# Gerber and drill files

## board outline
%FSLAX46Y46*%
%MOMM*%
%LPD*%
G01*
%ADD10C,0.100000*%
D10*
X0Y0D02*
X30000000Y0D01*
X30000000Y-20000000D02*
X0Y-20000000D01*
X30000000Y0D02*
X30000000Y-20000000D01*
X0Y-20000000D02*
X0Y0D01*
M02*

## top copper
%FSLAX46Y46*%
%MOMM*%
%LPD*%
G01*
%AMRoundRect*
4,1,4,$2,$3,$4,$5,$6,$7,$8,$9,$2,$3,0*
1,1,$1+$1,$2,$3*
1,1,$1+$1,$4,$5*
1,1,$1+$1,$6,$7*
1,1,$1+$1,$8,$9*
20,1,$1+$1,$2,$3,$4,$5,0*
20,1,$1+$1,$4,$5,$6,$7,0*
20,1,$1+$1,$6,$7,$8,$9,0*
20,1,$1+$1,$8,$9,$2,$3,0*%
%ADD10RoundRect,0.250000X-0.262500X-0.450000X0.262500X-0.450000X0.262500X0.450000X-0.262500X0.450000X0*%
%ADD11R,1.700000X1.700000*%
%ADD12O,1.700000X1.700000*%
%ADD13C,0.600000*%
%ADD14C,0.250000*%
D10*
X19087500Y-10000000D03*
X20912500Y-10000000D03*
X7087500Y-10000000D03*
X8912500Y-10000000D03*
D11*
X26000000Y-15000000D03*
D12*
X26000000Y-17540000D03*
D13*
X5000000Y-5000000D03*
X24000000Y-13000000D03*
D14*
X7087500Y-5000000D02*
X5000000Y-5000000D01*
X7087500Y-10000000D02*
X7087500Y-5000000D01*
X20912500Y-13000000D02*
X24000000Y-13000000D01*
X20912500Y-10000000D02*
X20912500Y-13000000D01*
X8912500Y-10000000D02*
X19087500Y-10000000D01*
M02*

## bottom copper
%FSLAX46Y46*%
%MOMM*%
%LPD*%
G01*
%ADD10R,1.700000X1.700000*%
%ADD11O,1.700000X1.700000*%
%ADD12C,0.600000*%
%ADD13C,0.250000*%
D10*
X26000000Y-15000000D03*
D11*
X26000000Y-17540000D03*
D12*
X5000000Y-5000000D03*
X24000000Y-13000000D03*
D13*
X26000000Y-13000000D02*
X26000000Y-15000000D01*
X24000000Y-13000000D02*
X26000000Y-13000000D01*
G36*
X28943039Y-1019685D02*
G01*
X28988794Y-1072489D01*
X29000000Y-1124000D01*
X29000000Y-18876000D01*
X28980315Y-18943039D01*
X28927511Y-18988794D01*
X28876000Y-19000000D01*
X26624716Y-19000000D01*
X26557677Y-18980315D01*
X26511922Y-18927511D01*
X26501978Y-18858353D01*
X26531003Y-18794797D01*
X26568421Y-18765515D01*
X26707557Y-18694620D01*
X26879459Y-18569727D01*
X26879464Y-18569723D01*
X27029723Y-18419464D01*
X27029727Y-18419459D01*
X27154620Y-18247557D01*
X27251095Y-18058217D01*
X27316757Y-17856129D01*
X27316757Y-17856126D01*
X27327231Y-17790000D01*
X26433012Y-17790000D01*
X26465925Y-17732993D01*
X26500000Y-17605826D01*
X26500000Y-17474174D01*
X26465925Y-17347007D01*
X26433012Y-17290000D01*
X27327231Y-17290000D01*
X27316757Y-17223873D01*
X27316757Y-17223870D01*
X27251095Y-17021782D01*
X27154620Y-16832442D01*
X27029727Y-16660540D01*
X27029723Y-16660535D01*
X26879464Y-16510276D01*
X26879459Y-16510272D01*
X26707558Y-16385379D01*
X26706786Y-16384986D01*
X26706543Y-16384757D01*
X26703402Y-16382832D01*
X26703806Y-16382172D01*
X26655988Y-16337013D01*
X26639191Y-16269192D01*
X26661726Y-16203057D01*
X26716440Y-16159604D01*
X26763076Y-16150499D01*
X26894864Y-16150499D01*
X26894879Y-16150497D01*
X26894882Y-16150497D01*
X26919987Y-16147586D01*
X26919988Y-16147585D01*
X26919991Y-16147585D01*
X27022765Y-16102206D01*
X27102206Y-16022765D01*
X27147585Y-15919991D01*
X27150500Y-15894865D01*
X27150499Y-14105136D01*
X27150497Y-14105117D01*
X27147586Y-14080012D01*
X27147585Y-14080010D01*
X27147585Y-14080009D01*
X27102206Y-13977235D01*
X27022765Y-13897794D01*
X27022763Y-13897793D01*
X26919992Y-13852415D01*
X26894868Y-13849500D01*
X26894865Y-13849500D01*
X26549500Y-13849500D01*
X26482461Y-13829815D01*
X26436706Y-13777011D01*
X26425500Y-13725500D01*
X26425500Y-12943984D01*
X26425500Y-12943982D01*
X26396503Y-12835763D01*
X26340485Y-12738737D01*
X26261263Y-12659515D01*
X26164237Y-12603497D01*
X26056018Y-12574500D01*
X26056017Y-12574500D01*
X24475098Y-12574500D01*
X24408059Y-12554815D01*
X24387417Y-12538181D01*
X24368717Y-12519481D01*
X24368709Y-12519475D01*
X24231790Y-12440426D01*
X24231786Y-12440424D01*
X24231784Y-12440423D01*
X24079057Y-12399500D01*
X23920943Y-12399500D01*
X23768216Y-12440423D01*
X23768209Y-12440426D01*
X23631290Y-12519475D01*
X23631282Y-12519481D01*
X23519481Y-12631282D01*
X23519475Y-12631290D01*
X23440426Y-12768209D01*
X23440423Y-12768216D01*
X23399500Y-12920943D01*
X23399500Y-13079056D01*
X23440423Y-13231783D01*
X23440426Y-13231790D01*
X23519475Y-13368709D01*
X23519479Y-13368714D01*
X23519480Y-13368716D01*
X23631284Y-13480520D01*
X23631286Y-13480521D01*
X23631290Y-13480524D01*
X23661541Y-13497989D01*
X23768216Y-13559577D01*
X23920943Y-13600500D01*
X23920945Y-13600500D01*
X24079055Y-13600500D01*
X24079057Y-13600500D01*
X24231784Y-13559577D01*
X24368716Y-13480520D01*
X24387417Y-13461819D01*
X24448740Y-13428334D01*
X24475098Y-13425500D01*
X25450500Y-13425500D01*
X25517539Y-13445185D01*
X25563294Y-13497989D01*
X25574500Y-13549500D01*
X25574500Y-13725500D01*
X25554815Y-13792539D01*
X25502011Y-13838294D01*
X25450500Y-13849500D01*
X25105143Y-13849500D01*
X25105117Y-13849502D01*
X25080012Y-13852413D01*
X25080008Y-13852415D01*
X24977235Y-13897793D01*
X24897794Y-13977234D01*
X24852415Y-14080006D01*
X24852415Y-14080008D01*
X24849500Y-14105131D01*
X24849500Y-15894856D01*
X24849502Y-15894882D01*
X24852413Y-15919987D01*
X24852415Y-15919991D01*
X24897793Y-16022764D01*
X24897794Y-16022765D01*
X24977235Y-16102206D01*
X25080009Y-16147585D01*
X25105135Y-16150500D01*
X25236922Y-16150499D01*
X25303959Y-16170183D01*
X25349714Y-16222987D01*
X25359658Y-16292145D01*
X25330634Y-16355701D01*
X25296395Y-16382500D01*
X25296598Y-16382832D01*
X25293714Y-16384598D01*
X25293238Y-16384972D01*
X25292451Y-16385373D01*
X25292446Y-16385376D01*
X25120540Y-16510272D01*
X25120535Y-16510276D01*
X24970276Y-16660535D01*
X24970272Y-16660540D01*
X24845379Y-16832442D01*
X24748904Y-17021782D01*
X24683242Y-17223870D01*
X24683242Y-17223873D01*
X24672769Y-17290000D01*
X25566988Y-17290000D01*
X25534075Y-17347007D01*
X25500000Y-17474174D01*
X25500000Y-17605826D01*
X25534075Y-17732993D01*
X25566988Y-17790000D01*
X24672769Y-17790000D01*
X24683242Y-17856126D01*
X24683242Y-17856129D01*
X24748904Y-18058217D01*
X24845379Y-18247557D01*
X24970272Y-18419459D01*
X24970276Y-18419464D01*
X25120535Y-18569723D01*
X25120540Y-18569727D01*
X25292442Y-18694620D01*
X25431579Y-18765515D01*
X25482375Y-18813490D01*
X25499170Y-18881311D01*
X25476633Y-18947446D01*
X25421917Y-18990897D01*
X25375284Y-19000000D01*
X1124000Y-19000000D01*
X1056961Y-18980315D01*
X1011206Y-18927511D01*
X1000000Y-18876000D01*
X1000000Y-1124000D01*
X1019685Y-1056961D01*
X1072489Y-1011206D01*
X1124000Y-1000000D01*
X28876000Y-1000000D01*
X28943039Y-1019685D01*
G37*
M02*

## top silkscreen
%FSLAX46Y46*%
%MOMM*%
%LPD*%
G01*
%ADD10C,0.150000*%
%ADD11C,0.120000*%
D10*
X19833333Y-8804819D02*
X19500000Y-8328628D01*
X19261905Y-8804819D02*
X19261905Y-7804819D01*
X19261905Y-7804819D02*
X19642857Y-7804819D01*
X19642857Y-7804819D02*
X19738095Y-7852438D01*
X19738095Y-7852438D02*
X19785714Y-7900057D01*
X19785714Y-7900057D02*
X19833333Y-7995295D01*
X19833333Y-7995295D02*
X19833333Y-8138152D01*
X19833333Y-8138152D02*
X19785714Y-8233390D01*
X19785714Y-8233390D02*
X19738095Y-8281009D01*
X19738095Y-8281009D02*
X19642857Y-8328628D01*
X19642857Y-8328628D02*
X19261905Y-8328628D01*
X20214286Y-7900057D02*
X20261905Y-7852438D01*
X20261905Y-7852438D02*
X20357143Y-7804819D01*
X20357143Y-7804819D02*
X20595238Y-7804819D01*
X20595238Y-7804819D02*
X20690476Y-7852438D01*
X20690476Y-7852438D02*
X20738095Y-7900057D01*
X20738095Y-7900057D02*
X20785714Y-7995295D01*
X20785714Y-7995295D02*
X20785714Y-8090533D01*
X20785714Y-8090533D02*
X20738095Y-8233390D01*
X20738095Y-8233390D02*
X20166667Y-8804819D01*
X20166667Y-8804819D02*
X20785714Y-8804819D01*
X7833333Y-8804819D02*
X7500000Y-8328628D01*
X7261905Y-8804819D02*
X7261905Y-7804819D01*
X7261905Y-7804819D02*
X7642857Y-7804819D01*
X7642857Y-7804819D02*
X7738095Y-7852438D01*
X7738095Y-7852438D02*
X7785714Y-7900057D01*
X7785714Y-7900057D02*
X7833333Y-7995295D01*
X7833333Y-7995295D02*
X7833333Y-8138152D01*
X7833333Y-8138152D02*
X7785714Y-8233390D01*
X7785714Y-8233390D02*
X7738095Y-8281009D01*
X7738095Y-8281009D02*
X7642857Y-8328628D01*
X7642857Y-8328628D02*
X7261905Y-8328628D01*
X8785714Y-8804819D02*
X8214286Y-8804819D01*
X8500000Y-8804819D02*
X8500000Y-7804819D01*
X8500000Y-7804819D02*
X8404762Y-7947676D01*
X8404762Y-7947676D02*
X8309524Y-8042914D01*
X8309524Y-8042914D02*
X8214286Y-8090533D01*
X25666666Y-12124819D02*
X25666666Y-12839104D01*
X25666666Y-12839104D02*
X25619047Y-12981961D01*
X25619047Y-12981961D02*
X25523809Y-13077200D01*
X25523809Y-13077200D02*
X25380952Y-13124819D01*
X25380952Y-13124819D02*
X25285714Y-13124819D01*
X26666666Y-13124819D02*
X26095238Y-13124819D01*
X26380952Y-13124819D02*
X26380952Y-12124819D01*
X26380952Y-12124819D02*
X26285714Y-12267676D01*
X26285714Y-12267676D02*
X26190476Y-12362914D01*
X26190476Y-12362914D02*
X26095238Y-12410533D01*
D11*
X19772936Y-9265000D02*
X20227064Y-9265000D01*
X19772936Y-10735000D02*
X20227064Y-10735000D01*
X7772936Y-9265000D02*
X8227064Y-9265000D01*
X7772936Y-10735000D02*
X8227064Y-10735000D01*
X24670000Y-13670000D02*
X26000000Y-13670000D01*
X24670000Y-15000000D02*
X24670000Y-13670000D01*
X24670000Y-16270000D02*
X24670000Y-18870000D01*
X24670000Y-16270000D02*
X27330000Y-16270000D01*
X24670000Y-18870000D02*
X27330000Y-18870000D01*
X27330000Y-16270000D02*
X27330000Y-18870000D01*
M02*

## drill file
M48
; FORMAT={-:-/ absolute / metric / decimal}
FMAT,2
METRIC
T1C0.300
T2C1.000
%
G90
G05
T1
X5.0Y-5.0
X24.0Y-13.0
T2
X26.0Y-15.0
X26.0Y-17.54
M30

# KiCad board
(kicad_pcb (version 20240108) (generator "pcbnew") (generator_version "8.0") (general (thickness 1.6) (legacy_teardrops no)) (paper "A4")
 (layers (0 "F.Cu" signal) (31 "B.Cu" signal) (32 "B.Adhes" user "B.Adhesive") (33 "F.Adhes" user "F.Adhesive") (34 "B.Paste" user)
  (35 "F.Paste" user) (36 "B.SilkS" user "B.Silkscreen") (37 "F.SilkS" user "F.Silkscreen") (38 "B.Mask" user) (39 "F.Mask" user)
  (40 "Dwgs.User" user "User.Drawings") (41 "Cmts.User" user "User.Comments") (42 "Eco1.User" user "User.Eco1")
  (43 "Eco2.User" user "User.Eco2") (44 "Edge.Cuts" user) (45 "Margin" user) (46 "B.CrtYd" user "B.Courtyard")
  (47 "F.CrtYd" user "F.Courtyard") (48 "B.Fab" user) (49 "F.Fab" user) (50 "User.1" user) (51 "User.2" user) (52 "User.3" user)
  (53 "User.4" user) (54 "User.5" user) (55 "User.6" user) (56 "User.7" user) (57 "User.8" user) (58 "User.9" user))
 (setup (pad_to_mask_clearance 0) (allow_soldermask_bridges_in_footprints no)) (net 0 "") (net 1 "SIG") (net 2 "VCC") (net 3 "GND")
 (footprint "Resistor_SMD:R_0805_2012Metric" (layer "F.Cu") (at 20 10)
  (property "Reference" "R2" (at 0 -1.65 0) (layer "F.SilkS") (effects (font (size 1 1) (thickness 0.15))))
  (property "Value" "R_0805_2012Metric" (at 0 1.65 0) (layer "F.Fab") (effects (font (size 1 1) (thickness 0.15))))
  (fp_line (start -0.227064 -0.735) (end 0.227064 -0.735) (stroke (width 0.12) (type solid)) (layer "F.SilkS"))
  (fp_line (start -0.227064 0.735) (end 0.227064 0.735) (stroke (width 0.12) (type solid)) (layer "F.SilkS"))
  (pad "1" smd roundrect (at -0.9125 0) (size 1.025 1.4) (layers "F.Cu" "F.Paste" "F.Mask") (roundrect_rratio 0.243902) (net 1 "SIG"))
  (pad "2" smd roundrect (at 0.9125 0) (size 1.025 1.4) (layers "F.Cu" "F.Paste" "F.Mask") (roundrect_rratio 0.243902) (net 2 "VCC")))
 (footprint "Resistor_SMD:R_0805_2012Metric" (layer "F.Cu") (at 8 10)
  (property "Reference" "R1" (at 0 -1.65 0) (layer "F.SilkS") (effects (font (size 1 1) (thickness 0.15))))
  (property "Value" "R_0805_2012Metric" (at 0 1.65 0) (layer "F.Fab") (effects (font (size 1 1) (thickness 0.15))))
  (fp_line (start -0.227064 -0.735) (end 0.227064 -0.735) (stroke (width 0.12) (type solid)) (layer "F.SilkS"))
  (fp_line (start -0.227064 0.735) (end 0.227064 0.735) (stroke (width 0.12) (type solid)) (layer "F.SilkS"))
  (pad "1" smd roundrect (at -0.9125 0) (size 1.025 1.4) (layers "F.Cu" "F.Paste" "F.Mask") (roundrect_rratio 0.243902) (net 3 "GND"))
  (pad "2" smd roundrect (at 0.9125 0) (size 1.025 1.4) (layers "F.Cu" "F.Paste" "F.Mask") (roundrect_rratio 0.243902) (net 1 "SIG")))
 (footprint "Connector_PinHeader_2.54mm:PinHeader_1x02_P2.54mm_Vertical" (layer "F.Cu") (at 26 15)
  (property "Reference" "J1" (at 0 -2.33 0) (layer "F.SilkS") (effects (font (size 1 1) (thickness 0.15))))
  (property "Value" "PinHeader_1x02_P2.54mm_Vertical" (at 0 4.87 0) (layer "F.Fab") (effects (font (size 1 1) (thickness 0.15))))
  (fp_line (start -1.33 -1.33) (end 0 -1.33) (stroke (width 0.12) (type solid)) (layer "F.SilkS"))
  (fp_line (start -1.33 0) (end -1.33 -1.33) (stroke (width 0.12) (type solid)) (layer "F.SilkS"))
  (fp_line (start -1.33 1.27) (end -1.33 3.87) (stroke (width 0.12) (type solid)) (layer "F.SilkS"))
  (fp_line (start -1.33 1.27) (end 1.33 1.27) (stroke (width 0.12) (type solid)) (layer "F.SilkS"))
  (fp_line (start -1.33 3.87) (end 1.33 3.87) (stroke (width 0.12) (type solid)) (layer "F.SilkS"))
  (fp_line (start 1.33 1.27) (end 1.33 3.87) (stroke (width 0.12) (type solid)) (layer "F.SilkS"))
  (pad "1" thru_hole rect (at 0 0) (size 1.7 1.7) (drill 1) (layers "*.Cu" "*.Mask") (remove_unused_layers no) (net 2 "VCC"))
  (pad "2" thru_hole oval (at 0 2.54) (size 1.7 1.7) (drill 1) (layers "*.Cu" "*.Mask") (remove_unused_layers no) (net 3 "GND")))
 (gr_line (start 0 0) (end 30 0) (stroke (width 0.1) (type default)) (layer "Edge.Cuts"))
 (gr_line (start 30 20) (end 0 20) (stroke (width 0.1) (type default)) (layer "Edge.Cuts"))
 (gr_line (start 30 0) (end 30 20) (stroke (width 0.1) (type default)) (layer "Edge.Cuts"))
 (gr_line (start 0 20) (end 0 0) (stroke (width 0.1) (type default)) (layer "Edge.Cuts"))
 (segment (start 7.0875 5) (end 5 5) (width 0.25) (layer "F.Cu") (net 3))
 (segment (start 7.0875 10) (end 7.0875 5) (width 0.25) (layer "F.Cu") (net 3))
 (via (at 5 5) (size 0.6) (drill 0.3) (layers "F.Cu" "B.Cu") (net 3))
 (segment (start 20.9125 13) (end 24 13) (width 0.25) (layer "F.Cu") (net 2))
 (segment (start 20.9125 10) (end 20.9125 13) (width 0.25) (layer "F.Cu") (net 2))
 (via (at 24 13) (size 0.6) (drill 0.3) (layers "F.Cu" "B.Cu") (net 2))
 (segment (start 26 13) (end 26 15) (width 0.25) (layer "B.Cu") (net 2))
 (segment (start 24 13) (end 26 13) (width 0.25) (layer "B.Cu") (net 2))
 (segment (start 8.9125 10) (end 19.0875 10) (width 0.25) (layer "F.Cu") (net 1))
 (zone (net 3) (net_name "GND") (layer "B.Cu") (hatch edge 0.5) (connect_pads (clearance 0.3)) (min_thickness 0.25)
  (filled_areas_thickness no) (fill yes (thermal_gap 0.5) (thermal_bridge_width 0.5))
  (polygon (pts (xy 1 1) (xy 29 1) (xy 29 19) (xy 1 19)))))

